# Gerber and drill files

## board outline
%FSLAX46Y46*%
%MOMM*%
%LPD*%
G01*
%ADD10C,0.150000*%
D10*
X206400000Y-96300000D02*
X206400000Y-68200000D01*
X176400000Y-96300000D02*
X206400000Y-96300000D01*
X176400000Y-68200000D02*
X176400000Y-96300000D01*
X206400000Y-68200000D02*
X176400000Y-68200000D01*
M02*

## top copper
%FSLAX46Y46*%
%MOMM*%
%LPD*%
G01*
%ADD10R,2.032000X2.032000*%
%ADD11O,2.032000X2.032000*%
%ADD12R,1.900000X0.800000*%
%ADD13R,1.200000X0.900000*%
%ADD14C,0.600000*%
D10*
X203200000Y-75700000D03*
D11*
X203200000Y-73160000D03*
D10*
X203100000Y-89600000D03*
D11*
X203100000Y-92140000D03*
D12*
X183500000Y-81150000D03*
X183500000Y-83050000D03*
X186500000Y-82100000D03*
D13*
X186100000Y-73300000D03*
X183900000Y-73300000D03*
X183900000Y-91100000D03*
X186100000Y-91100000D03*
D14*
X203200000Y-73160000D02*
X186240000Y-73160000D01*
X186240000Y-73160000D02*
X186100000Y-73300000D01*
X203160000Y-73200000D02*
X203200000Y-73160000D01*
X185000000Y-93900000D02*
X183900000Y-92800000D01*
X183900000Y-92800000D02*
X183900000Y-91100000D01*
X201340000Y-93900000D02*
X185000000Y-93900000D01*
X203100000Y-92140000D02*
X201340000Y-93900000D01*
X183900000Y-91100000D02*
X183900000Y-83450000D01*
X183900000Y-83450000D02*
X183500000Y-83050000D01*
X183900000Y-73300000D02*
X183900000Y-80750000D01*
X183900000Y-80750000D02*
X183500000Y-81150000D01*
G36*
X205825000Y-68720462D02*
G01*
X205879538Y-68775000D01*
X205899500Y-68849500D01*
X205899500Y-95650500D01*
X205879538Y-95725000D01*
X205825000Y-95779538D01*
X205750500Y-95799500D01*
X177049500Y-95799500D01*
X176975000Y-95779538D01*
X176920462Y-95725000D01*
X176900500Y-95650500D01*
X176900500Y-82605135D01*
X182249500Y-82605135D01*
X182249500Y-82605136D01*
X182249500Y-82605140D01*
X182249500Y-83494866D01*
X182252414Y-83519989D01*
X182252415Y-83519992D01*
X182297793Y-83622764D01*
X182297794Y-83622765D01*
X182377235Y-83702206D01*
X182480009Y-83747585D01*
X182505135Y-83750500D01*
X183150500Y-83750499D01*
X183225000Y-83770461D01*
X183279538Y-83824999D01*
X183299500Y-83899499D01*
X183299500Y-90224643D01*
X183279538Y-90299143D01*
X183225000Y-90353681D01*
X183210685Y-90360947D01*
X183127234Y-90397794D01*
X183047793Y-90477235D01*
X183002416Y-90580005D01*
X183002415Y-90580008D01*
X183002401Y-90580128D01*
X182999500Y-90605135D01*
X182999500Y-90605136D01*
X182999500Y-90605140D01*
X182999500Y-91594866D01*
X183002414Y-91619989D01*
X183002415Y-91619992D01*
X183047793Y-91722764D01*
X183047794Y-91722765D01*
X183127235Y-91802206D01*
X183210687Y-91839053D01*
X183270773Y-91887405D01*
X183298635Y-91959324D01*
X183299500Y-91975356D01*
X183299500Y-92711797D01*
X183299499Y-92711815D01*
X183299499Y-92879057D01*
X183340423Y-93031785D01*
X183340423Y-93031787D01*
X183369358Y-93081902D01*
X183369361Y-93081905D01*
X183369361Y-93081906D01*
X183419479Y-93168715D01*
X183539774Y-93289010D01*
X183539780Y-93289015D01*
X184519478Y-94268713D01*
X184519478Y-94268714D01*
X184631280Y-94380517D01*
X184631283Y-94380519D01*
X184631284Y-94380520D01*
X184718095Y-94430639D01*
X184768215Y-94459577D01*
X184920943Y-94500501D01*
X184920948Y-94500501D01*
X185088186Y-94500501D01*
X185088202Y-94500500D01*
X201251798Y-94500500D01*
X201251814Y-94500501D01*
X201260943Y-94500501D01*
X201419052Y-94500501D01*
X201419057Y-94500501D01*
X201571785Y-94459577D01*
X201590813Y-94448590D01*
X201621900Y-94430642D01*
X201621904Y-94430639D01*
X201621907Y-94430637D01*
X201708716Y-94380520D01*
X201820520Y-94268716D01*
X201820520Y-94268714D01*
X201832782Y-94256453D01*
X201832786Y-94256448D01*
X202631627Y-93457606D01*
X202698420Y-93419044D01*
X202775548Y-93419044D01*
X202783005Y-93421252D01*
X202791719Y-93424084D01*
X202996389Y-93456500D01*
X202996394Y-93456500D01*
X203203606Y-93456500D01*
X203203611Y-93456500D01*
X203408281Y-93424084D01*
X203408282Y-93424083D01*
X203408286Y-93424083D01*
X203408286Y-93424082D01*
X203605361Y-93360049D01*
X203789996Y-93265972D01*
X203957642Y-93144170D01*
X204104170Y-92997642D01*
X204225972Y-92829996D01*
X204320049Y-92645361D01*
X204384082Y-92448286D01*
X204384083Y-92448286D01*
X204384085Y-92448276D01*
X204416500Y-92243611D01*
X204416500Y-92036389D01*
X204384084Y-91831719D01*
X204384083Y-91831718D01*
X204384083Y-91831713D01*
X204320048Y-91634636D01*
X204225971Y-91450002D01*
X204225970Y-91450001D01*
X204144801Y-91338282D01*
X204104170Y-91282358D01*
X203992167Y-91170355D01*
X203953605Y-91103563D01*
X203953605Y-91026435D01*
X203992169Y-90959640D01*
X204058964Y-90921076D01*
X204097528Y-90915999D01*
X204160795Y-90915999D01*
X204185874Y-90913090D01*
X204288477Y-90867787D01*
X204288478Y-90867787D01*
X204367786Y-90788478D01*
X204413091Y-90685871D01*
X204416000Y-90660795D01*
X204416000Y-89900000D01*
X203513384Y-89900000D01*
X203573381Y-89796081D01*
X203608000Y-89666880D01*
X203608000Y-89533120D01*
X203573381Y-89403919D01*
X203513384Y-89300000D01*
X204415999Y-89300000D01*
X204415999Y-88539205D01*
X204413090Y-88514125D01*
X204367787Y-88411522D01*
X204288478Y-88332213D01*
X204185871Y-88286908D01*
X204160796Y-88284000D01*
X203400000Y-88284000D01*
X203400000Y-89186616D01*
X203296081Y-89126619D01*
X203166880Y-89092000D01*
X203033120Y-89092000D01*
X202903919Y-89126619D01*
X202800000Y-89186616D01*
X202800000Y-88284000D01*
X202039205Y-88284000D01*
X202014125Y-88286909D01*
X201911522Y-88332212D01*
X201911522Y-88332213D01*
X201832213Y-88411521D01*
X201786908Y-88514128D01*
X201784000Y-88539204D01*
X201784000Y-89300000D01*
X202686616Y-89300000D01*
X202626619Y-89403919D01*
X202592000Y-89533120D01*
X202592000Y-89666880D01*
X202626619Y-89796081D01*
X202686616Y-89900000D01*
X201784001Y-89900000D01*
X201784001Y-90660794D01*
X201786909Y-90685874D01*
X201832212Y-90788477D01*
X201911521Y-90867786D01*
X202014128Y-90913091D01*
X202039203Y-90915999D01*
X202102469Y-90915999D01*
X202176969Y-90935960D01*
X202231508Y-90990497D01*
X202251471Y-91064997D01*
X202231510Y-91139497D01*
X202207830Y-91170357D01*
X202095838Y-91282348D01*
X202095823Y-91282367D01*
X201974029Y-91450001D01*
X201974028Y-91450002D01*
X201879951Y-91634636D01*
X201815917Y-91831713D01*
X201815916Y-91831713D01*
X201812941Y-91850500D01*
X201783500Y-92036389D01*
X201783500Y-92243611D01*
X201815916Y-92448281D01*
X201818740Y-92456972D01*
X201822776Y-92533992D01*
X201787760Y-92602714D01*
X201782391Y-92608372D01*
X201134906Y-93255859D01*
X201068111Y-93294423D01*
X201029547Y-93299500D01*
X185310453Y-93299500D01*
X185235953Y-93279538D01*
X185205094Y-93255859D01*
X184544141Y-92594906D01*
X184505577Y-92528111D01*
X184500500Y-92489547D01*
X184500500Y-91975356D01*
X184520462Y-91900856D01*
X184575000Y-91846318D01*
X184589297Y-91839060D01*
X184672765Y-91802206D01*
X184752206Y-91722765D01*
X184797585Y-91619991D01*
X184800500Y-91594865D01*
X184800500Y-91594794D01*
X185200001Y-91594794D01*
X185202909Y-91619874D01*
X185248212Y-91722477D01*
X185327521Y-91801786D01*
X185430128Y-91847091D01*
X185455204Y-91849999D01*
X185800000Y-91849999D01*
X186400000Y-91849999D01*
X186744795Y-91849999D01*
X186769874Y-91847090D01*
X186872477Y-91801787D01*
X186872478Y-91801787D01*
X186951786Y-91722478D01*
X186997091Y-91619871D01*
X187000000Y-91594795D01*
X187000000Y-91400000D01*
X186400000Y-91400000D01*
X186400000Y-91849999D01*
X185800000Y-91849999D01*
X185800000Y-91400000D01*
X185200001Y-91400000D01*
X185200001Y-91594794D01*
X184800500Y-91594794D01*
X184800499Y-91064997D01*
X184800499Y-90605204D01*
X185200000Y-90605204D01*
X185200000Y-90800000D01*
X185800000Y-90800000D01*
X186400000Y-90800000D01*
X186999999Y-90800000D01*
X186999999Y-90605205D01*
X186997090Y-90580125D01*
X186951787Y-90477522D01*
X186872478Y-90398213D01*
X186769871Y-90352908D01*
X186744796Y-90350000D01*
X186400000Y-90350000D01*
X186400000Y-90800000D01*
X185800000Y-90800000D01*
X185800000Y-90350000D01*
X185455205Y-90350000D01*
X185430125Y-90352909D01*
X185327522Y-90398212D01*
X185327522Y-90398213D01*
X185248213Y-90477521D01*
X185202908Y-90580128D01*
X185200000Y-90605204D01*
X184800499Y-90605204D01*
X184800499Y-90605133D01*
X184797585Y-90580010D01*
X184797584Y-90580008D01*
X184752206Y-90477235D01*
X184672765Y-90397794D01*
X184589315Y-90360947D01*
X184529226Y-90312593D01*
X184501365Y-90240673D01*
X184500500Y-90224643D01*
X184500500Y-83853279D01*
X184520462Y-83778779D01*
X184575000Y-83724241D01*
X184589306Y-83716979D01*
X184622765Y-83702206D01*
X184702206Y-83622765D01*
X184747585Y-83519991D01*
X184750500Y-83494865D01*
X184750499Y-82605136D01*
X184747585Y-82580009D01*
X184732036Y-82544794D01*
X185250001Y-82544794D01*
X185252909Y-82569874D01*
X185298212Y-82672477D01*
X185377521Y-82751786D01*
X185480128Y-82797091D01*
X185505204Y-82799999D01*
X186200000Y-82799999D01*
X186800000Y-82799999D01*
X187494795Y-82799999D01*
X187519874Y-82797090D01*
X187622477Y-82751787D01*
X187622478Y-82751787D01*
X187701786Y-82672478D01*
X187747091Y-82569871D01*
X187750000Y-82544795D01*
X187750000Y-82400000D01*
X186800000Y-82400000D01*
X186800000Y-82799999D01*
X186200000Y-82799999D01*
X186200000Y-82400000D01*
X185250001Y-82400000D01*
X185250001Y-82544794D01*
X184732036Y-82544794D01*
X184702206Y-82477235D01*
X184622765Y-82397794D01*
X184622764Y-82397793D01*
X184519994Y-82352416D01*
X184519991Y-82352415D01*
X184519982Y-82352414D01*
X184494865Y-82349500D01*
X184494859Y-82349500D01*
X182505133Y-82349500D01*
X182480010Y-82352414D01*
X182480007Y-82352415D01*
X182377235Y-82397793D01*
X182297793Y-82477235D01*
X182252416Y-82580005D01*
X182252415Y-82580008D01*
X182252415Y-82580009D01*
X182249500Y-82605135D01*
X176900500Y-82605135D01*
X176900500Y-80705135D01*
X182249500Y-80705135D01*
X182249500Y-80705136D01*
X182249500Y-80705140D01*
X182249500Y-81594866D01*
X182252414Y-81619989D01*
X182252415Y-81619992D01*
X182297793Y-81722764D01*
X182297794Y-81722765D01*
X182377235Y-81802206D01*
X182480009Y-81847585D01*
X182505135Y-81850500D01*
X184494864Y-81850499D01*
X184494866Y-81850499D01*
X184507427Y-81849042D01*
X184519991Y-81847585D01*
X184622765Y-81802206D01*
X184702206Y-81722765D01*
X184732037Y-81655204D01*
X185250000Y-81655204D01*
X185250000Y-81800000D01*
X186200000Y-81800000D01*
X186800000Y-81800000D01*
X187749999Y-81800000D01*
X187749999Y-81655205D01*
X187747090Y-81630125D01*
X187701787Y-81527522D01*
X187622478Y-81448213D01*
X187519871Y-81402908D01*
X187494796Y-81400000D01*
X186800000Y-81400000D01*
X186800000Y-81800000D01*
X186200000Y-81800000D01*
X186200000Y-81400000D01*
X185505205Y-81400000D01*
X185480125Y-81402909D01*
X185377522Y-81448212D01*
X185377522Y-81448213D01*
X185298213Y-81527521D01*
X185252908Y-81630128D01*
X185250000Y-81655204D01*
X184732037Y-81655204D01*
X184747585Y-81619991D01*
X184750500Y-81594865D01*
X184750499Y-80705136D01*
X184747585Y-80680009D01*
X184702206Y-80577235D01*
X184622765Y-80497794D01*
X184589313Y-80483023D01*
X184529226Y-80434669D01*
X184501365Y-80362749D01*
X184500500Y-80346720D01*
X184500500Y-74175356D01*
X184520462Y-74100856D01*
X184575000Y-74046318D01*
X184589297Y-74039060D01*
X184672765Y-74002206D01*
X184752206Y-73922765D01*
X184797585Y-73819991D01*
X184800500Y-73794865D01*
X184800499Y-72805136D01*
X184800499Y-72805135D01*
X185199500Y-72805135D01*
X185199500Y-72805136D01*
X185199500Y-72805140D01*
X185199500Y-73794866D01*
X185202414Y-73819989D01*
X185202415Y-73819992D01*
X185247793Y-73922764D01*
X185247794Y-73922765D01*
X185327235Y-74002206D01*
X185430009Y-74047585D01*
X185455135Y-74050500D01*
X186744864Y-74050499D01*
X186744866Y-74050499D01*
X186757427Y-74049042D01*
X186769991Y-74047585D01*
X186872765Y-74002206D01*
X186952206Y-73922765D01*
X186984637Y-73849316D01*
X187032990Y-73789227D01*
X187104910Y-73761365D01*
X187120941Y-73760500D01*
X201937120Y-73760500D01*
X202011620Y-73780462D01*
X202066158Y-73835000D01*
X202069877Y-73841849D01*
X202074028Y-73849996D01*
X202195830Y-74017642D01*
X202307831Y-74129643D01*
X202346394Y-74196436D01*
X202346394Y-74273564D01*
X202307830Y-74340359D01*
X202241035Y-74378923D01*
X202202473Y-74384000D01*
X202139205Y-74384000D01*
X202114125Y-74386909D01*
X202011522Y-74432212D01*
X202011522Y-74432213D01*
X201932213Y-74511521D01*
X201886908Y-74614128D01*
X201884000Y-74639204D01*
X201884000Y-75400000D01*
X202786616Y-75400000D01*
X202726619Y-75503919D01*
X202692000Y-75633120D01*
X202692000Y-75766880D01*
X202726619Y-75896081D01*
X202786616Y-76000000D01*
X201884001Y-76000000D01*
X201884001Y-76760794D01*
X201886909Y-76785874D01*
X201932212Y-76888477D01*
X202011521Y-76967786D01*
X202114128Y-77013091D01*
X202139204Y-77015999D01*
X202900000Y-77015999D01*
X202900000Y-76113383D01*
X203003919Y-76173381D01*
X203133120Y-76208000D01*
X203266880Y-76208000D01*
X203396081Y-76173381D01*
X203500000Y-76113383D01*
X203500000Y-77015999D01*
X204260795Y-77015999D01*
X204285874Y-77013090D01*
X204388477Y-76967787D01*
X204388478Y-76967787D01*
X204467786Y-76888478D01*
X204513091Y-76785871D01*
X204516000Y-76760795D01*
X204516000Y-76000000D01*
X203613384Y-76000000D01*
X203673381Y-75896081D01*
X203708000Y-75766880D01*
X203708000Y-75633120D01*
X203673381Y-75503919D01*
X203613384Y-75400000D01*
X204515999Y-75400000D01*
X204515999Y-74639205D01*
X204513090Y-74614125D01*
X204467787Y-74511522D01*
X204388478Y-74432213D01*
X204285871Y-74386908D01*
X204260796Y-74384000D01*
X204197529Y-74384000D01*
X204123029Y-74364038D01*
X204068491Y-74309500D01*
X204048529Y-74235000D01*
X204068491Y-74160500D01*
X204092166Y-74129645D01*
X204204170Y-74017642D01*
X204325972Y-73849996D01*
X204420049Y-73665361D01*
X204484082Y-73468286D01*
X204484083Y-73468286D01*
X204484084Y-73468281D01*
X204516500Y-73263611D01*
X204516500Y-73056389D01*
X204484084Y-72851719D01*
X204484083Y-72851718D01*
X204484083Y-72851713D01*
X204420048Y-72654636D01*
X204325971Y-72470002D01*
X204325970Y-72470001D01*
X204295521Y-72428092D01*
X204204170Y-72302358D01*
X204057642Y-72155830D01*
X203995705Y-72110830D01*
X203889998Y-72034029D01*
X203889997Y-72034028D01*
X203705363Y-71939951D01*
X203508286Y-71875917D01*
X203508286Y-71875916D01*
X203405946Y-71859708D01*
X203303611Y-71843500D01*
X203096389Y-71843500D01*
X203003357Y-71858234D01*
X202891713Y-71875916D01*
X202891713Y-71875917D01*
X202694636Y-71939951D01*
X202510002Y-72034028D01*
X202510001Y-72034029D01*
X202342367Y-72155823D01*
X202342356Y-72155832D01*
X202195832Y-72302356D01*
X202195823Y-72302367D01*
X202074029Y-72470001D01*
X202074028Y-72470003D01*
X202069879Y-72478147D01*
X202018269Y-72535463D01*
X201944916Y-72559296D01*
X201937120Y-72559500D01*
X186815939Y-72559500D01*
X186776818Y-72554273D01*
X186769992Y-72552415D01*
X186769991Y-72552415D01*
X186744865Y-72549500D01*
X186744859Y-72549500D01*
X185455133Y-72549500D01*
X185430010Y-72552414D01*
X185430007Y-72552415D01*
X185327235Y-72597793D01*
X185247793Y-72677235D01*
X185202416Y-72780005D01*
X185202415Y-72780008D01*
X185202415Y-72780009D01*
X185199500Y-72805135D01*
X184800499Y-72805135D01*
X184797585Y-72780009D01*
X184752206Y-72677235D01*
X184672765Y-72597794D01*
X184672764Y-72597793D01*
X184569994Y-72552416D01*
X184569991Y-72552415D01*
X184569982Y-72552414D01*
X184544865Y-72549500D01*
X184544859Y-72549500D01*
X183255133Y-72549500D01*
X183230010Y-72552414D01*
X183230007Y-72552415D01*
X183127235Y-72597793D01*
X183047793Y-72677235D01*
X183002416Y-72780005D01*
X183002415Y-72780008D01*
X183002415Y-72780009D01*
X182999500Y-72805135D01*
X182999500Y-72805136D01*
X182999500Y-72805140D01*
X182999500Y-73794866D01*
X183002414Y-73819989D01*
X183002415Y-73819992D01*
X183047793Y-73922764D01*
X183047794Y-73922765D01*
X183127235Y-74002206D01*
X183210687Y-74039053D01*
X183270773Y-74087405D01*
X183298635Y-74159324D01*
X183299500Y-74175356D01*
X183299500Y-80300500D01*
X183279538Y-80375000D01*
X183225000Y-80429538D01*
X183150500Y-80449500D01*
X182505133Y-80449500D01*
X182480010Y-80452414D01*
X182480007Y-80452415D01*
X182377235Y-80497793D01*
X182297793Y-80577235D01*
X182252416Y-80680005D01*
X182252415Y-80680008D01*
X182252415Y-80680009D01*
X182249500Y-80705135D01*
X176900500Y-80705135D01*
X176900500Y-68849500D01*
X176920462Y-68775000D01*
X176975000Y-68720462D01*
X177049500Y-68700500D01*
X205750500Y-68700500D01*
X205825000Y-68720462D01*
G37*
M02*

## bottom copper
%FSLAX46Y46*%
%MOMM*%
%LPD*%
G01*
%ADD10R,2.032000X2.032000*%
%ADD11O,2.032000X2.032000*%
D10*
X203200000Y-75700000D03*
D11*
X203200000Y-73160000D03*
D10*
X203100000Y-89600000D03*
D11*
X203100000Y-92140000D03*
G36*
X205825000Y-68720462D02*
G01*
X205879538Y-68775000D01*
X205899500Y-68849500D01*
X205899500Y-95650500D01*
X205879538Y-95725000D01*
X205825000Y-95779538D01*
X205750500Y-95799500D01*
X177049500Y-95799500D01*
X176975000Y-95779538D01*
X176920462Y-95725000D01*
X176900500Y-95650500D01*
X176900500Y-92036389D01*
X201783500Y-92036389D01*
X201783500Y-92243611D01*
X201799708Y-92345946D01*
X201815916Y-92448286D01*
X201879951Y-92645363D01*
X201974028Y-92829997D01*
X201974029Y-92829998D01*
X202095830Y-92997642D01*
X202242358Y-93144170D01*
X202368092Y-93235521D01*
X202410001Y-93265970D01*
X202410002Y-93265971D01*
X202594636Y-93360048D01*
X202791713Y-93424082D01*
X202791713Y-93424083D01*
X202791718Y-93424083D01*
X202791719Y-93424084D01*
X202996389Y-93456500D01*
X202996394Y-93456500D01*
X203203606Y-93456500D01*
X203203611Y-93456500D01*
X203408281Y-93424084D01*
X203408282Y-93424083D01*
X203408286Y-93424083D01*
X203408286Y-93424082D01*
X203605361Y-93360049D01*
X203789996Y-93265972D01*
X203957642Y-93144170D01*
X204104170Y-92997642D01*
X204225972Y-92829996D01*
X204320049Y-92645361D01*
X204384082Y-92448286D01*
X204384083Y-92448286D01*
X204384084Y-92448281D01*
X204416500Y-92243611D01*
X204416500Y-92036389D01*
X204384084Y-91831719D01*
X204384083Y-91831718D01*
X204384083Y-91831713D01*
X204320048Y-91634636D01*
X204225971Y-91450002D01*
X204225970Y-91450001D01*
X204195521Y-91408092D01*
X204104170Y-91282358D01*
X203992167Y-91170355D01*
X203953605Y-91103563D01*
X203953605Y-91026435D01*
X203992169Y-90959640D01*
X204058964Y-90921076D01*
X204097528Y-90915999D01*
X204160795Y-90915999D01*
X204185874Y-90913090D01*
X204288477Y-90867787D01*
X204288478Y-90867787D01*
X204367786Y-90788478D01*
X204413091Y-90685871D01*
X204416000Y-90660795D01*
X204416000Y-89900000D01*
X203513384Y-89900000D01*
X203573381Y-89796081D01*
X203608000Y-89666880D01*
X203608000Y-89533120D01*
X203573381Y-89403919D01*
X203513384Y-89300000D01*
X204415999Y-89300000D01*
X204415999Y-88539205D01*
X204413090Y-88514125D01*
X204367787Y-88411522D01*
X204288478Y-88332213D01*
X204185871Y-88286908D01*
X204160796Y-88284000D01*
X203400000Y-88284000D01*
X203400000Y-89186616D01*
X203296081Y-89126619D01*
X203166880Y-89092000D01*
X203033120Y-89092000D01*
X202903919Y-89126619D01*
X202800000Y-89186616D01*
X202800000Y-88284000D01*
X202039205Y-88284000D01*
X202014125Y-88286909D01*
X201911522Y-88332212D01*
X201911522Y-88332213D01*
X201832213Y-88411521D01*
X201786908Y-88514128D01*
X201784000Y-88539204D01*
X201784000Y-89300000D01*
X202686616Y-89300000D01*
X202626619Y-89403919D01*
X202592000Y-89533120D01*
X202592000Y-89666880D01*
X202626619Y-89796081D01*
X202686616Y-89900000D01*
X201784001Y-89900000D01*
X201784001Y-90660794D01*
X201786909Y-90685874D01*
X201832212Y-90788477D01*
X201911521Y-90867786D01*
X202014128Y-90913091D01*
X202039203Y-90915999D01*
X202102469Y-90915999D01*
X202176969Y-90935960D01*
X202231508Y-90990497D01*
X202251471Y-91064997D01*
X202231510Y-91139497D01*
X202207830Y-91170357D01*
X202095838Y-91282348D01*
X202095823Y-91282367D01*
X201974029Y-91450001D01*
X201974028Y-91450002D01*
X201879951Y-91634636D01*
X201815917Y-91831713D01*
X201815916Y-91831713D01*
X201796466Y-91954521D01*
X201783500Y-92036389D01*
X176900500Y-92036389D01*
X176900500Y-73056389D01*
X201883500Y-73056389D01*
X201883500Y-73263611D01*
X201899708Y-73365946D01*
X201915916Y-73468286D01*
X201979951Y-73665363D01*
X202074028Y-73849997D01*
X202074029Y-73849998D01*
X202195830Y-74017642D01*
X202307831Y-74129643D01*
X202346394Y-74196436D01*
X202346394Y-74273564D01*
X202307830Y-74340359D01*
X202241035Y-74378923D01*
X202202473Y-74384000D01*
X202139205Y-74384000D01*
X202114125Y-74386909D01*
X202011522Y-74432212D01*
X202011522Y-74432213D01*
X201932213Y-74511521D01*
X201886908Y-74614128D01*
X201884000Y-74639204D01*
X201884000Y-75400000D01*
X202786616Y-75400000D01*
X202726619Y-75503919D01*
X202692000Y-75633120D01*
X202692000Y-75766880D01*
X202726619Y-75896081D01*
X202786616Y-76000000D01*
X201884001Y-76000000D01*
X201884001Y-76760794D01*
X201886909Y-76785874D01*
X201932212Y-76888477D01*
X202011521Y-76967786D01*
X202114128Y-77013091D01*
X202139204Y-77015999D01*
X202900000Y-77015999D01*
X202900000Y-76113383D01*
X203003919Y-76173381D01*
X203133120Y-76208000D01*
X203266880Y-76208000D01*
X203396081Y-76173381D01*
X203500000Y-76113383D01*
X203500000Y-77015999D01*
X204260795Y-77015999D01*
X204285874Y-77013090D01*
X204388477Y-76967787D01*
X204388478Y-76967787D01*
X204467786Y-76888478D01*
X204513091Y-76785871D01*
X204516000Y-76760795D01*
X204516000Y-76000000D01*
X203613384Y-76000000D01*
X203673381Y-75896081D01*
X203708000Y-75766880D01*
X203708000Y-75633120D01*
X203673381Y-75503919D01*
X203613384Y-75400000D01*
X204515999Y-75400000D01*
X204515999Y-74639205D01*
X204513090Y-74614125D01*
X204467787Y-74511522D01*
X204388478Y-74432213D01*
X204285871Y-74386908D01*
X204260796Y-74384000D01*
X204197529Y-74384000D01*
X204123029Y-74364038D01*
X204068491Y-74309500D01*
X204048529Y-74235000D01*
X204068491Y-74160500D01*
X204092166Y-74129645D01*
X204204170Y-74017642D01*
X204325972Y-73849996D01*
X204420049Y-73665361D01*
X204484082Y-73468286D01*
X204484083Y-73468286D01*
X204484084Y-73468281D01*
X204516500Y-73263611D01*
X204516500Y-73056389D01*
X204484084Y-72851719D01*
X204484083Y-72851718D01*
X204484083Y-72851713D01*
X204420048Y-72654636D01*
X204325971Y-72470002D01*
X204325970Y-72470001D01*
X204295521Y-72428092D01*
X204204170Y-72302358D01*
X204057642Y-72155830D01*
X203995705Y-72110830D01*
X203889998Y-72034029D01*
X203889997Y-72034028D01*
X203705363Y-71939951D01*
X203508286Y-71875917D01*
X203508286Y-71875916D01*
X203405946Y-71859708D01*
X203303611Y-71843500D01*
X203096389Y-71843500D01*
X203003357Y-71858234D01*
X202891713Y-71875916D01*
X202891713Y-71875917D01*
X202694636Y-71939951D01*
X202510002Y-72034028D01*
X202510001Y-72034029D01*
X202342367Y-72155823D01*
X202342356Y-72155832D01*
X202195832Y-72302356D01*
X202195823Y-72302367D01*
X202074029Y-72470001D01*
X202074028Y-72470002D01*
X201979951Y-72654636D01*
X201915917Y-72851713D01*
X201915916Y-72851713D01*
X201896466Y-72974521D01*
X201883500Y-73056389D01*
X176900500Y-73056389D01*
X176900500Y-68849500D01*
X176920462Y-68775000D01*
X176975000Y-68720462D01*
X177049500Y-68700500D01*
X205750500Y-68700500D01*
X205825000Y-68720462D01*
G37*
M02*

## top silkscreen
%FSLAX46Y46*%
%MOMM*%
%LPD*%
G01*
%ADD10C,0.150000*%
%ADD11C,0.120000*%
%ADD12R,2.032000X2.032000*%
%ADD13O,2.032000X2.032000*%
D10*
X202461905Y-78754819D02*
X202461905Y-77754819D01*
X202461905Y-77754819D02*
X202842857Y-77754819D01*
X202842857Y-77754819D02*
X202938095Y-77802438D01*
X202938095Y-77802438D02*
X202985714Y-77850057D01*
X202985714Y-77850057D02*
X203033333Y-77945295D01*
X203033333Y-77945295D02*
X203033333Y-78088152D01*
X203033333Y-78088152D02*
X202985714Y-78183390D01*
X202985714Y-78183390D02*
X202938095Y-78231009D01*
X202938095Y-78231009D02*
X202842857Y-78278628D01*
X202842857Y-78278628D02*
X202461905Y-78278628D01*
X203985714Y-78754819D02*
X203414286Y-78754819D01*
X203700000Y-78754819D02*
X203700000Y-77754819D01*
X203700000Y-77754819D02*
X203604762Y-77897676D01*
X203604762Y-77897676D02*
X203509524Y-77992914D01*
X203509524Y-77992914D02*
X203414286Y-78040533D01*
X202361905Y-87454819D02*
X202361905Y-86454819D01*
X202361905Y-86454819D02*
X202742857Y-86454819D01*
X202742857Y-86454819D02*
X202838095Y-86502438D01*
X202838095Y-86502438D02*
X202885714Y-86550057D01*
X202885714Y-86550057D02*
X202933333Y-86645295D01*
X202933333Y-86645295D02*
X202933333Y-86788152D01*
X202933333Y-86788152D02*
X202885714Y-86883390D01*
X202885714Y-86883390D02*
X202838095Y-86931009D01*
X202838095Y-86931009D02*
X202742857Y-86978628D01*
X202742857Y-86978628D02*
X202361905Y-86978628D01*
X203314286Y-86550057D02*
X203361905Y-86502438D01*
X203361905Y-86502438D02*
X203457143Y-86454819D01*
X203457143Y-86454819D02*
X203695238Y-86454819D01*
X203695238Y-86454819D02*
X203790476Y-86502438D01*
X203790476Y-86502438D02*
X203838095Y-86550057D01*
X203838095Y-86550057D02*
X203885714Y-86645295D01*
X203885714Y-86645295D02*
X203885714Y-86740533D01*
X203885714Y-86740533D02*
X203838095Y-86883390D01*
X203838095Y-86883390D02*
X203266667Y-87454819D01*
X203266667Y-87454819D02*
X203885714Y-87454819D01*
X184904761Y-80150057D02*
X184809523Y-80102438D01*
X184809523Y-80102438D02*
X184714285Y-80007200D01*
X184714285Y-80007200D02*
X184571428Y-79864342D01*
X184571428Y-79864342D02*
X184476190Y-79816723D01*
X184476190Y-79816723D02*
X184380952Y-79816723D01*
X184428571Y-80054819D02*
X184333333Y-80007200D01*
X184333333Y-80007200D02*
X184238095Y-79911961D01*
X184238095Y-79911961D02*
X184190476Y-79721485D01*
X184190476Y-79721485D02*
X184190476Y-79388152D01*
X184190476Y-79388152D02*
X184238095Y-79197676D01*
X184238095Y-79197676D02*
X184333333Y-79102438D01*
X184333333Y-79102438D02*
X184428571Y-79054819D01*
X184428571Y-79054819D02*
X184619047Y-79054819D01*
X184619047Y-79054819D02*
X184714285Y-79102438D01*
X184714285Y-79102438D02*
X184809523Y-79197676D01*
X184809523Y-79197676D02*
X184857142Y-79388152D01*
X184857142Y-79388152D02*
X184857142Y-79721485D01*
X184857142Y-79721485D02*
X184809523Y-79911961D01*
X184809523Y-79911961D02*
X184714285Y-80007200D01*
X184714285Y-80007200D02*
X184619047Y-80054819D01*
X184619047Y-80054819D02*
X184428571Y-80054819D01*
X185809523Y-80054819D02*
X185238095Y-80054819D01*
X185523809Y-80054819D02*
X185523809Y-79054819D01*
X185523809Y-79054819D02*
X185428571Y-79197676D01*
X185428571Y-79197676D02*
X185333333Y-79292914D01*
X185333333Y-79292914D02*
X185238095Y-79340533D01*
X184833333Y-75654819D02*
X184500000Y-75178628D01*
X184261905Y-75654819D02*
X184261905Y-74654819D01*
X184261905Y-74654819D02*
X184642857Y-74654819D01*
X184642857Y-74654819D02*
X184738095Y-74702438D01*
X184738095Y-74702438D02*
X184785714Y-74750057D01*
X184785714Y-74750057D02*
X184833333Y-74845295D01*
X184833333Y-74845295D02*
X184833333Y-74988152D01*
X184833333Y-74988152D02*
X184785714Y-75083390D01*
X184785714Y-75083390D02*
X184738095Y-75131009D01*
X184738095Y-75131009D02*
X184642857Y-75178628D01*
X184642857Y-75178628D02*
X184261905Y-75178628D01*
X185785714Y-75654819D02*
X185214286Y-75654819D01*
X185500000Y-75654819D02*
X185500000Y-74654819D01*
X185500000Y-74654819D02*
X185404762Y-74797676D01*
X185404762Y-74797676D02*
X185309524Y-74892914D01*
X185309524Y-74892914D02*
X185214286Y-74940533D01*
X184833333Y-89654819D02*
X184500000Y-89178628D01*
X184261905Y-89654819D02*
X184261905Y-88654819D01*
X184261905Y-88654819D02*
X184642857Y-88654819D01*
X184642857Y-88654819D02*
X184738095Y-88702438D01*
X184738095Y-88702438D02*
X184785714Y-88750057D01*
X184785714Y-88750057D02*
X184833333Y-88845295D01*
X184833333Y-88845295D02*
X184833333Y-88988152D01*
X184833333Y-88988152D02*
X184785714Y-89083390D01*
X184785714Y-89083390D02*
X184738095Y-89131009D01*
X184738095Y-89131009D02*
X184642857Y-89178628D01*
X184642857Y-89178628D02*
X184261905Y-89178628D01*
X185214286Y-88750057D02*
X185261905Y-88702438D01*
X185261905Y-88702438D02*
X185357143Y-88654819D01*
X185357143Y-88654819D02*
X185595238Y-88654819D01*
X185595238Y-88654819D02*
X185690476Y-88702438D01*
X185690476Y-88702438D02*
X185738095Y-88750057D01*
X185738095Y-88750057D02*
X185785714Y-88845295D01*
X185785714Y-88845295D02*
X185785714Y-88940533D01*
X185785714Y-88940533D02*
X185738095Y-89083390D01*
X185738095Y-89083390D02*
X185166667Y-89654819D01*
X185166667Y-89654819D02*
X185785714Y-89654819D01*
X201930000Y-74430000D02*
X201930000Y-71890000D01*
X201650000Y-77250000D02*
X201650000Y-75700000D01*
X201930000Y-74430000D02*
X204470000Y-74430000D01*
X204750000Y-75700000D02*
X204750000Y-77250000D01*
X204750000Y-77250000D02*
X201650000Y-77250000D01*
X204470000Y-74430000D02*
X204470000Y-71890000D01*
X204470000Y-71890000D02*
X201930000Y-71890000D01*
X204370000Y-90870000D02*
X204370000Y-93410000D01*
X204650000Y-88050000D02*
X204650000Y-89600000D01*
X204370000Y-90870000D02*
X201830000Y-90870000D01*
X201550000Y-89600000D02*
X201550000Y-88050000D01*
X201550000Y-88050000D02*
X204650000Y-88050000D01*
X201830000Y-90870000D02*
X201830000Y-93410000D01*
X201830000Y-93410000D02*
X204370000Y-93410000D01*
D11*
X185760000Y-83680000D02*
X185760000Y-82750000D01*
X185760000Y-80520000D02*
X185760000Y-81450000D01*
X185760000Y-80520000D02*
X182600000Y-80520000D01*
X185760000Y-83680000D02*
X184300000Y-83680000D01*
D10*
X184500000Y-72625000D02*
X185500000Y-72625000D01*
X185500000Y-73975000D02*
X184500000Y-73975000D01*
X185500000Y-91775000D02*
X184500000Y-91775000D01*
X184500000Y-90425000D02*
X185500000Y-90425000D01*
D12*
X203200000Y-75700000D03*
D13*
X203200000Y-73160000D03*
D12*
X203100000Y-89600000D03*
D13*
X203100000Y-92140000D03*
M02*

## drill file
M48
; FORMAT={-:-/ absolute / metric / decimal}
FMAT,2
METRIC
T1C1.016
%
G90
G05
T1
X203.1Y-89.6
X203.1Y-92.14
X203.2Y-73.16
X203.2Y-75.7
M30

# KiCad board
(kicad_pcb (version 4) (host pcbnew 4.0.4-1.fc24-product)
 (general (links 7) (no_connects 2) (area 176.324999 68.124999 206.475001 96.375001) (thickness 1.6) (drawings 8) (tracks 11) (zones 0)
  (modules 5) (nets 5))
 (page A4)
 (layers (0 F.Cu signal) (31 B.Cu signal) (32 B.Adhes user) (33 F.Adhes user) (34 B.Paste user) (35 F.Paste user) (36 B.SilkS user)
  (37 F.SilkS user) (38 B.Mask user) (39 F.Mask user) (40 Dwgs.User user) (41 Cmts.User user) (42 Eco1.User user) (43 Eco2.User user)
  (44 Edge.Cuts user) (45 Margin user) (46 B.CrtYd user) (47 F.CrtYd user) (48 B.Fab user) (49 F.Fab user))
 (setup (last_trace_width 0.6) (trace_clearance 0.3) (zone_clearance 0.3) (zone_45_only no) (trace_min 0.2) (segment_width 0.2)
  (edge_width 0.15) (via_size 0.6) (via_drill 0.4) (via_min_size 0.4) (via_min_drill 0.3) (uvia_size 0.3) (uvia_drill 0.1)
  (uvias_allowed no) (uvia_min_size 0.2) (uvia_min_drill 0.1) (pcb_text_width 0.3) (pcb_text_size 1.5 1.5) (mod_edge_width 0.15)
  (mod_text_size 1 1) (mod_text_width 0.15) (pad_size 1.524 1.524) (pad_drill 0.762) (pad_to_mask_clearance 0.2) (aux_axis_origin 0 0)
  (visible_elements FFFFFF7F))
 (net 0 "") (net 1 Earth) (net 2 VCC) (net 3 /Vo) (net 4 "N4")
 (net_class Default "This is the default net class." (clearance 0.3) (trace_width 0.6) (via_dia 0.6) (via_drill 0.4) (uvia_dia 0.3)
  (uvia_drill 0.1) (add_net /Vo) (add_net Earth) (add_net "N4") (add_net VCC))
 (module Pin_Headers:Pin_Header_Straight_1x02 (layer F.Cu) (at 203.2 75.7 180)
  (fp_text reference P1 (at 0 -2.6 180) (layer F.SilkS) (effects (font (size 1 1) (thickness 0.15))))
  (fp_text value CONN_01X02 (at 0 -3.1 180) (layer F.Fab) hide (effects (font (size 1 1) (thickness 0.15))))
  (fp_line (start 1.27 1.27) (end 1.27 3.81) (layer F.SilkS) (width 0.15))
  (fp_line (start 1.55 -1.55) (end 1.55 0) (layer F.SilkS) (width 0.15))
  (fp_line (start 1.27 1.27) (end -1.27 1.27) (layer F.SilkS) (width 0.15))
  (fp_line (start -1.55 0) (end -1.55 -1.55) (layer F.SilkS) (width 0.15))
  (fp_line (start -1.55 -1.55) (end 1.55 -1.55) (layer F.SilkS) (width 0.15))
  (fp_line (start -1.27 1.27) (end -1.27 3.81) (layer F.SilkS) (width 0.15))
  (fp_line (start -1.27 3.81) (end 1.27 3.81) (layer F.SilkS) (width 0.15))
  (pad 1 thru_hole rect (at 0 0 180) (size 2.032 2.032) (drill 1.016) (layers *.Cu *.Mask F.SilkS) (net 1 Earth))
  (pad 2 thru_hole oval (at 0 2.54 180) (size 2.032 2.032) (drill 1.016) (layers *.Cu *.Mask F.SilkS) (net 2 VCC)))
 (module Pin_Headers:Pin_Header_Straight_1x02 (layer F.Cu) (at 203.1 89.6)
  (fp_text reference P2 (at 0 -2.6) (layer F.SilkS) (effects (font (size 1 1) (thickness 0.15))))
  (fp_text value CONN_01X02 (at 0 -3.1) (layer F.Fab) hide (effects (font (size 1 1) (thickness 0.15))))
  (fp_line (start 1.27 1.27) (end 1.27 3.81) (layer F.SilkS) (width 0.15))
  (fp_line (start 1.55 -1.55) (end 1.55 0) (layer F.SilkS) (width 0.15))
  (fp_line (start 1.27 1.27) (end -1.27 1.27) (layer F.SilkS) (width 0.15))
  (fp_line (start -1.55 0) (end -1.55 -1.55) (layer F.SilkS) (width 0.15))
  (fp_line (start -1.55 -1.55) (end 1.55 -1.55) (layer F.SilkS) (width 0.15))
  (fp_line (start -1.27 1.27) (end -1.27 3.81) (layer F.SilkS) (width 0.15))
  (fp_line (start -1.27 3.81) (end 1.27 3.81) (layer F.SilkS) (width 0.15))
  (pad 1 thru_hole rect (at 0 0) (size 2.032 2.032) (drill 1.016) (layers *.Cu *.Mask F.SilkS) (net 1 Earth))
  (pad 2 thru_hole oval (at 0 2.54) (size 2.032 2.032) (drill 1.016) (layers *.Cu *.Mask F.SilkS) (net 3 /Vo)))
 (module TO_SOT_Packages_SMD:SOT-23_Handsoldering (layer F.Cu) (at 185 82.1)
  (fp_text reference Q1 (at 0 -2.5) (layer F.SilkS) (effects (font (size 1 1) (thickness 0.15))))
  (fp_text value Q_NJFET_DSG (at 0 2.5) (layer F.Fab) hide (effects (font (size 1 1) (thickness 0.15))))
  (fp_line (start 0.76 1.58) (end 0.76 0.65) (layer F.SilkS) (width 0.12))
  (fp_line (start 0.76 -1.58) (end 0.76 -0.65) (layer F.SilkS) (width 0.12))
  (fp_line (start 0.76 -1.58) (end -2.4 -1.58) (layer F.SilkS) (width 0.12))
  (fp_line (start 0.76 1.58) (end -0.7 1.58) (layer F.SilkS) (width 0.12))
  (pad 1 smd rect (at -1.5 -0.95) (size 1.9 0.8) (layers F.Cu F.Paste F.Mask) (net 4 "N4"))
  (pad 2 smd rect (at -1.5 0.95) (size 1.9 0.8) (layers F.Cu F.Paste F.Mask) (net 3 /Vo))
  (pad 3 smd rect (at 1.5 0) (size 1.9 0.8) (layers F.Cu F.Paste F.Mask) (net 1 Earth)))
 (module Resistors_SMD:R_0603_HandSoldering (layer F.Cu) (at 185 73.3 180)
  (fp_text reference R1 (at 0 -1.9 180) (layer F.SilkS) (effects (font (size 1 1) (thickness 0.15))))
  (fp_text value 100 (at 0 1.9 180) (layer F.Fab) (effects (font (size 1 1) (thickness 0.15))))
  (fp_line (start 0.5 0.675) (end -0.5 0.675) (layer F.SilkS) (width 0.15))
  (fp_line (start -0.5 -0.675) (end 0.5 -0.675) (layer F.SilkS) (width 0.15))
  (pad 1 smd rect (at -1.1 0 180) (size 1.2 0.9) (layers F.Cu F.Paste F.Mask) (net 2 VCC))
  (pad 2 smd rect (at 1.1 0 180) (size 1.2 0.9) (layers F.Cu F.Paste F.Mask) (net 4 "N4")))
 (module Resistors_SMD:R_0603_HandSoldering (layer F.Cu) (at 185 91.1)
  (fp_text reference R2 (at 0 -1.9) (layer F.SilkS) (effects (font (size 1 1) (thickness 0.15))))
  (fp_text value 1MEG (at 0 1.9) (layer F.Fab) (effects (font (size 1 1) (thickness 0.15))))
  (fp_line (start 0.5 0.675) (end -0.5 0.675) (layer F.SilkS) (width 0.15))
  (fp_line (start -0.5 -0.675) (end 0.5 -0.675) (layer F.SilkS) (width 0.15))
  (pad 1 smd rect (at -1.1 0) (size 1.2 0.9) (layers F.Cu F.Paste F.Mask) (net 3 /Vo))
  (pad 2 smd rect (at 1.1 0) (size 1.2 0.9) (layers F.Cu F.Paste F.Mask) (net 1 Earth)))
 (gr_line (start 206.4 96.3) (end 206.4 68.2) (angle 90) (layer Edge.Cuts) (width 0.15))
 (gr_line (start 176.4 96.3) (end 206.4 96.3) (angle 90) (layer Edge.Cuts) (width 0.15))
 (gr_line (start 176.4 68.2) (end 176.4 96.3) (angle 90) (layer Edge.Cuts) (width 0.15))
 (gr_line (start 206.4 68.2) (end 176.4 68.2) (angle 90) (layer Edge.Cuts) (width 0.15))
 (segment (start 203.2 73.16) (end 186.24 73.16) (width 0.6) (layer F.Cu) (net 2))
 (segment (start 186.24 73.16) (end 186.1 73.3) (width 0.6) (layer F.Cu) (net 2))
 (segment (start 203.16 73.2) (end 203.2 73.16) (width 0.6) (layer F.Cu) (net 2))
 (segment (start 185 93.9) (end 183.9 92.8) (width 0.6) (layer F.Cu) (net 3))
 (segment (start 183.9 92.8) (end 183.9 91.1) (width 0.6) (layer F.Cu) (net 3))
 (segment (start 201.34 93.9) (end 185 93.9) (width 0.6) (layer F.Cu) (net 3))
 (segment (start 203.1 92.14) (end 201.34 93.9) (width 0.6) (layer F.Cu) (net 3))
 (segment (start 183.9 91.1) (end 183.9 83.45) (width 0.6) (layer F.Cu) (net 3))
 (segment (start 183.9 83.45) (end 183.5 83.05) (width 0.6) (layer F.Cu) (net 3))
 (segment (start 183.9 73.3) (end 183.9 80.75) (width 0.6) (layer F.Cu) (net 4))
 (segment (start 183.9 80.75) (end 183.5 81.15) (width 0.6) (layer F.Cu) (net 4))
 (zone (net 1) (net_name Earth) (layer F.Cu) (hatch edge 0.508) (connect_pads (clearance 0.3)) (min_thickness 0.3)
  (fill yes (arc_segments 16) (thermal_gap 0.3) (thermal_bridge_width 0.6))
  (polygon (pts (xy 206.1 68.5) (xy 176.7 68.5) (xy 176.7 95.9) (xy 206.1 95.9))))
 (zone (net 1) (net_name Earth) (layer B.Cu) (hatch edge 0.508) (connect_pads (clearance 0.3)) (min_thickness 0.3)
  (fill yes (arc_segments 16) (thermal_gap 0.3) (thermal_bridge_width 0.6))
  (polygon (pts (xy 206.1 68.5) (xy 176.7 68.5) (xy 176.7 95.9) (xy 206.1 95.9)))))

